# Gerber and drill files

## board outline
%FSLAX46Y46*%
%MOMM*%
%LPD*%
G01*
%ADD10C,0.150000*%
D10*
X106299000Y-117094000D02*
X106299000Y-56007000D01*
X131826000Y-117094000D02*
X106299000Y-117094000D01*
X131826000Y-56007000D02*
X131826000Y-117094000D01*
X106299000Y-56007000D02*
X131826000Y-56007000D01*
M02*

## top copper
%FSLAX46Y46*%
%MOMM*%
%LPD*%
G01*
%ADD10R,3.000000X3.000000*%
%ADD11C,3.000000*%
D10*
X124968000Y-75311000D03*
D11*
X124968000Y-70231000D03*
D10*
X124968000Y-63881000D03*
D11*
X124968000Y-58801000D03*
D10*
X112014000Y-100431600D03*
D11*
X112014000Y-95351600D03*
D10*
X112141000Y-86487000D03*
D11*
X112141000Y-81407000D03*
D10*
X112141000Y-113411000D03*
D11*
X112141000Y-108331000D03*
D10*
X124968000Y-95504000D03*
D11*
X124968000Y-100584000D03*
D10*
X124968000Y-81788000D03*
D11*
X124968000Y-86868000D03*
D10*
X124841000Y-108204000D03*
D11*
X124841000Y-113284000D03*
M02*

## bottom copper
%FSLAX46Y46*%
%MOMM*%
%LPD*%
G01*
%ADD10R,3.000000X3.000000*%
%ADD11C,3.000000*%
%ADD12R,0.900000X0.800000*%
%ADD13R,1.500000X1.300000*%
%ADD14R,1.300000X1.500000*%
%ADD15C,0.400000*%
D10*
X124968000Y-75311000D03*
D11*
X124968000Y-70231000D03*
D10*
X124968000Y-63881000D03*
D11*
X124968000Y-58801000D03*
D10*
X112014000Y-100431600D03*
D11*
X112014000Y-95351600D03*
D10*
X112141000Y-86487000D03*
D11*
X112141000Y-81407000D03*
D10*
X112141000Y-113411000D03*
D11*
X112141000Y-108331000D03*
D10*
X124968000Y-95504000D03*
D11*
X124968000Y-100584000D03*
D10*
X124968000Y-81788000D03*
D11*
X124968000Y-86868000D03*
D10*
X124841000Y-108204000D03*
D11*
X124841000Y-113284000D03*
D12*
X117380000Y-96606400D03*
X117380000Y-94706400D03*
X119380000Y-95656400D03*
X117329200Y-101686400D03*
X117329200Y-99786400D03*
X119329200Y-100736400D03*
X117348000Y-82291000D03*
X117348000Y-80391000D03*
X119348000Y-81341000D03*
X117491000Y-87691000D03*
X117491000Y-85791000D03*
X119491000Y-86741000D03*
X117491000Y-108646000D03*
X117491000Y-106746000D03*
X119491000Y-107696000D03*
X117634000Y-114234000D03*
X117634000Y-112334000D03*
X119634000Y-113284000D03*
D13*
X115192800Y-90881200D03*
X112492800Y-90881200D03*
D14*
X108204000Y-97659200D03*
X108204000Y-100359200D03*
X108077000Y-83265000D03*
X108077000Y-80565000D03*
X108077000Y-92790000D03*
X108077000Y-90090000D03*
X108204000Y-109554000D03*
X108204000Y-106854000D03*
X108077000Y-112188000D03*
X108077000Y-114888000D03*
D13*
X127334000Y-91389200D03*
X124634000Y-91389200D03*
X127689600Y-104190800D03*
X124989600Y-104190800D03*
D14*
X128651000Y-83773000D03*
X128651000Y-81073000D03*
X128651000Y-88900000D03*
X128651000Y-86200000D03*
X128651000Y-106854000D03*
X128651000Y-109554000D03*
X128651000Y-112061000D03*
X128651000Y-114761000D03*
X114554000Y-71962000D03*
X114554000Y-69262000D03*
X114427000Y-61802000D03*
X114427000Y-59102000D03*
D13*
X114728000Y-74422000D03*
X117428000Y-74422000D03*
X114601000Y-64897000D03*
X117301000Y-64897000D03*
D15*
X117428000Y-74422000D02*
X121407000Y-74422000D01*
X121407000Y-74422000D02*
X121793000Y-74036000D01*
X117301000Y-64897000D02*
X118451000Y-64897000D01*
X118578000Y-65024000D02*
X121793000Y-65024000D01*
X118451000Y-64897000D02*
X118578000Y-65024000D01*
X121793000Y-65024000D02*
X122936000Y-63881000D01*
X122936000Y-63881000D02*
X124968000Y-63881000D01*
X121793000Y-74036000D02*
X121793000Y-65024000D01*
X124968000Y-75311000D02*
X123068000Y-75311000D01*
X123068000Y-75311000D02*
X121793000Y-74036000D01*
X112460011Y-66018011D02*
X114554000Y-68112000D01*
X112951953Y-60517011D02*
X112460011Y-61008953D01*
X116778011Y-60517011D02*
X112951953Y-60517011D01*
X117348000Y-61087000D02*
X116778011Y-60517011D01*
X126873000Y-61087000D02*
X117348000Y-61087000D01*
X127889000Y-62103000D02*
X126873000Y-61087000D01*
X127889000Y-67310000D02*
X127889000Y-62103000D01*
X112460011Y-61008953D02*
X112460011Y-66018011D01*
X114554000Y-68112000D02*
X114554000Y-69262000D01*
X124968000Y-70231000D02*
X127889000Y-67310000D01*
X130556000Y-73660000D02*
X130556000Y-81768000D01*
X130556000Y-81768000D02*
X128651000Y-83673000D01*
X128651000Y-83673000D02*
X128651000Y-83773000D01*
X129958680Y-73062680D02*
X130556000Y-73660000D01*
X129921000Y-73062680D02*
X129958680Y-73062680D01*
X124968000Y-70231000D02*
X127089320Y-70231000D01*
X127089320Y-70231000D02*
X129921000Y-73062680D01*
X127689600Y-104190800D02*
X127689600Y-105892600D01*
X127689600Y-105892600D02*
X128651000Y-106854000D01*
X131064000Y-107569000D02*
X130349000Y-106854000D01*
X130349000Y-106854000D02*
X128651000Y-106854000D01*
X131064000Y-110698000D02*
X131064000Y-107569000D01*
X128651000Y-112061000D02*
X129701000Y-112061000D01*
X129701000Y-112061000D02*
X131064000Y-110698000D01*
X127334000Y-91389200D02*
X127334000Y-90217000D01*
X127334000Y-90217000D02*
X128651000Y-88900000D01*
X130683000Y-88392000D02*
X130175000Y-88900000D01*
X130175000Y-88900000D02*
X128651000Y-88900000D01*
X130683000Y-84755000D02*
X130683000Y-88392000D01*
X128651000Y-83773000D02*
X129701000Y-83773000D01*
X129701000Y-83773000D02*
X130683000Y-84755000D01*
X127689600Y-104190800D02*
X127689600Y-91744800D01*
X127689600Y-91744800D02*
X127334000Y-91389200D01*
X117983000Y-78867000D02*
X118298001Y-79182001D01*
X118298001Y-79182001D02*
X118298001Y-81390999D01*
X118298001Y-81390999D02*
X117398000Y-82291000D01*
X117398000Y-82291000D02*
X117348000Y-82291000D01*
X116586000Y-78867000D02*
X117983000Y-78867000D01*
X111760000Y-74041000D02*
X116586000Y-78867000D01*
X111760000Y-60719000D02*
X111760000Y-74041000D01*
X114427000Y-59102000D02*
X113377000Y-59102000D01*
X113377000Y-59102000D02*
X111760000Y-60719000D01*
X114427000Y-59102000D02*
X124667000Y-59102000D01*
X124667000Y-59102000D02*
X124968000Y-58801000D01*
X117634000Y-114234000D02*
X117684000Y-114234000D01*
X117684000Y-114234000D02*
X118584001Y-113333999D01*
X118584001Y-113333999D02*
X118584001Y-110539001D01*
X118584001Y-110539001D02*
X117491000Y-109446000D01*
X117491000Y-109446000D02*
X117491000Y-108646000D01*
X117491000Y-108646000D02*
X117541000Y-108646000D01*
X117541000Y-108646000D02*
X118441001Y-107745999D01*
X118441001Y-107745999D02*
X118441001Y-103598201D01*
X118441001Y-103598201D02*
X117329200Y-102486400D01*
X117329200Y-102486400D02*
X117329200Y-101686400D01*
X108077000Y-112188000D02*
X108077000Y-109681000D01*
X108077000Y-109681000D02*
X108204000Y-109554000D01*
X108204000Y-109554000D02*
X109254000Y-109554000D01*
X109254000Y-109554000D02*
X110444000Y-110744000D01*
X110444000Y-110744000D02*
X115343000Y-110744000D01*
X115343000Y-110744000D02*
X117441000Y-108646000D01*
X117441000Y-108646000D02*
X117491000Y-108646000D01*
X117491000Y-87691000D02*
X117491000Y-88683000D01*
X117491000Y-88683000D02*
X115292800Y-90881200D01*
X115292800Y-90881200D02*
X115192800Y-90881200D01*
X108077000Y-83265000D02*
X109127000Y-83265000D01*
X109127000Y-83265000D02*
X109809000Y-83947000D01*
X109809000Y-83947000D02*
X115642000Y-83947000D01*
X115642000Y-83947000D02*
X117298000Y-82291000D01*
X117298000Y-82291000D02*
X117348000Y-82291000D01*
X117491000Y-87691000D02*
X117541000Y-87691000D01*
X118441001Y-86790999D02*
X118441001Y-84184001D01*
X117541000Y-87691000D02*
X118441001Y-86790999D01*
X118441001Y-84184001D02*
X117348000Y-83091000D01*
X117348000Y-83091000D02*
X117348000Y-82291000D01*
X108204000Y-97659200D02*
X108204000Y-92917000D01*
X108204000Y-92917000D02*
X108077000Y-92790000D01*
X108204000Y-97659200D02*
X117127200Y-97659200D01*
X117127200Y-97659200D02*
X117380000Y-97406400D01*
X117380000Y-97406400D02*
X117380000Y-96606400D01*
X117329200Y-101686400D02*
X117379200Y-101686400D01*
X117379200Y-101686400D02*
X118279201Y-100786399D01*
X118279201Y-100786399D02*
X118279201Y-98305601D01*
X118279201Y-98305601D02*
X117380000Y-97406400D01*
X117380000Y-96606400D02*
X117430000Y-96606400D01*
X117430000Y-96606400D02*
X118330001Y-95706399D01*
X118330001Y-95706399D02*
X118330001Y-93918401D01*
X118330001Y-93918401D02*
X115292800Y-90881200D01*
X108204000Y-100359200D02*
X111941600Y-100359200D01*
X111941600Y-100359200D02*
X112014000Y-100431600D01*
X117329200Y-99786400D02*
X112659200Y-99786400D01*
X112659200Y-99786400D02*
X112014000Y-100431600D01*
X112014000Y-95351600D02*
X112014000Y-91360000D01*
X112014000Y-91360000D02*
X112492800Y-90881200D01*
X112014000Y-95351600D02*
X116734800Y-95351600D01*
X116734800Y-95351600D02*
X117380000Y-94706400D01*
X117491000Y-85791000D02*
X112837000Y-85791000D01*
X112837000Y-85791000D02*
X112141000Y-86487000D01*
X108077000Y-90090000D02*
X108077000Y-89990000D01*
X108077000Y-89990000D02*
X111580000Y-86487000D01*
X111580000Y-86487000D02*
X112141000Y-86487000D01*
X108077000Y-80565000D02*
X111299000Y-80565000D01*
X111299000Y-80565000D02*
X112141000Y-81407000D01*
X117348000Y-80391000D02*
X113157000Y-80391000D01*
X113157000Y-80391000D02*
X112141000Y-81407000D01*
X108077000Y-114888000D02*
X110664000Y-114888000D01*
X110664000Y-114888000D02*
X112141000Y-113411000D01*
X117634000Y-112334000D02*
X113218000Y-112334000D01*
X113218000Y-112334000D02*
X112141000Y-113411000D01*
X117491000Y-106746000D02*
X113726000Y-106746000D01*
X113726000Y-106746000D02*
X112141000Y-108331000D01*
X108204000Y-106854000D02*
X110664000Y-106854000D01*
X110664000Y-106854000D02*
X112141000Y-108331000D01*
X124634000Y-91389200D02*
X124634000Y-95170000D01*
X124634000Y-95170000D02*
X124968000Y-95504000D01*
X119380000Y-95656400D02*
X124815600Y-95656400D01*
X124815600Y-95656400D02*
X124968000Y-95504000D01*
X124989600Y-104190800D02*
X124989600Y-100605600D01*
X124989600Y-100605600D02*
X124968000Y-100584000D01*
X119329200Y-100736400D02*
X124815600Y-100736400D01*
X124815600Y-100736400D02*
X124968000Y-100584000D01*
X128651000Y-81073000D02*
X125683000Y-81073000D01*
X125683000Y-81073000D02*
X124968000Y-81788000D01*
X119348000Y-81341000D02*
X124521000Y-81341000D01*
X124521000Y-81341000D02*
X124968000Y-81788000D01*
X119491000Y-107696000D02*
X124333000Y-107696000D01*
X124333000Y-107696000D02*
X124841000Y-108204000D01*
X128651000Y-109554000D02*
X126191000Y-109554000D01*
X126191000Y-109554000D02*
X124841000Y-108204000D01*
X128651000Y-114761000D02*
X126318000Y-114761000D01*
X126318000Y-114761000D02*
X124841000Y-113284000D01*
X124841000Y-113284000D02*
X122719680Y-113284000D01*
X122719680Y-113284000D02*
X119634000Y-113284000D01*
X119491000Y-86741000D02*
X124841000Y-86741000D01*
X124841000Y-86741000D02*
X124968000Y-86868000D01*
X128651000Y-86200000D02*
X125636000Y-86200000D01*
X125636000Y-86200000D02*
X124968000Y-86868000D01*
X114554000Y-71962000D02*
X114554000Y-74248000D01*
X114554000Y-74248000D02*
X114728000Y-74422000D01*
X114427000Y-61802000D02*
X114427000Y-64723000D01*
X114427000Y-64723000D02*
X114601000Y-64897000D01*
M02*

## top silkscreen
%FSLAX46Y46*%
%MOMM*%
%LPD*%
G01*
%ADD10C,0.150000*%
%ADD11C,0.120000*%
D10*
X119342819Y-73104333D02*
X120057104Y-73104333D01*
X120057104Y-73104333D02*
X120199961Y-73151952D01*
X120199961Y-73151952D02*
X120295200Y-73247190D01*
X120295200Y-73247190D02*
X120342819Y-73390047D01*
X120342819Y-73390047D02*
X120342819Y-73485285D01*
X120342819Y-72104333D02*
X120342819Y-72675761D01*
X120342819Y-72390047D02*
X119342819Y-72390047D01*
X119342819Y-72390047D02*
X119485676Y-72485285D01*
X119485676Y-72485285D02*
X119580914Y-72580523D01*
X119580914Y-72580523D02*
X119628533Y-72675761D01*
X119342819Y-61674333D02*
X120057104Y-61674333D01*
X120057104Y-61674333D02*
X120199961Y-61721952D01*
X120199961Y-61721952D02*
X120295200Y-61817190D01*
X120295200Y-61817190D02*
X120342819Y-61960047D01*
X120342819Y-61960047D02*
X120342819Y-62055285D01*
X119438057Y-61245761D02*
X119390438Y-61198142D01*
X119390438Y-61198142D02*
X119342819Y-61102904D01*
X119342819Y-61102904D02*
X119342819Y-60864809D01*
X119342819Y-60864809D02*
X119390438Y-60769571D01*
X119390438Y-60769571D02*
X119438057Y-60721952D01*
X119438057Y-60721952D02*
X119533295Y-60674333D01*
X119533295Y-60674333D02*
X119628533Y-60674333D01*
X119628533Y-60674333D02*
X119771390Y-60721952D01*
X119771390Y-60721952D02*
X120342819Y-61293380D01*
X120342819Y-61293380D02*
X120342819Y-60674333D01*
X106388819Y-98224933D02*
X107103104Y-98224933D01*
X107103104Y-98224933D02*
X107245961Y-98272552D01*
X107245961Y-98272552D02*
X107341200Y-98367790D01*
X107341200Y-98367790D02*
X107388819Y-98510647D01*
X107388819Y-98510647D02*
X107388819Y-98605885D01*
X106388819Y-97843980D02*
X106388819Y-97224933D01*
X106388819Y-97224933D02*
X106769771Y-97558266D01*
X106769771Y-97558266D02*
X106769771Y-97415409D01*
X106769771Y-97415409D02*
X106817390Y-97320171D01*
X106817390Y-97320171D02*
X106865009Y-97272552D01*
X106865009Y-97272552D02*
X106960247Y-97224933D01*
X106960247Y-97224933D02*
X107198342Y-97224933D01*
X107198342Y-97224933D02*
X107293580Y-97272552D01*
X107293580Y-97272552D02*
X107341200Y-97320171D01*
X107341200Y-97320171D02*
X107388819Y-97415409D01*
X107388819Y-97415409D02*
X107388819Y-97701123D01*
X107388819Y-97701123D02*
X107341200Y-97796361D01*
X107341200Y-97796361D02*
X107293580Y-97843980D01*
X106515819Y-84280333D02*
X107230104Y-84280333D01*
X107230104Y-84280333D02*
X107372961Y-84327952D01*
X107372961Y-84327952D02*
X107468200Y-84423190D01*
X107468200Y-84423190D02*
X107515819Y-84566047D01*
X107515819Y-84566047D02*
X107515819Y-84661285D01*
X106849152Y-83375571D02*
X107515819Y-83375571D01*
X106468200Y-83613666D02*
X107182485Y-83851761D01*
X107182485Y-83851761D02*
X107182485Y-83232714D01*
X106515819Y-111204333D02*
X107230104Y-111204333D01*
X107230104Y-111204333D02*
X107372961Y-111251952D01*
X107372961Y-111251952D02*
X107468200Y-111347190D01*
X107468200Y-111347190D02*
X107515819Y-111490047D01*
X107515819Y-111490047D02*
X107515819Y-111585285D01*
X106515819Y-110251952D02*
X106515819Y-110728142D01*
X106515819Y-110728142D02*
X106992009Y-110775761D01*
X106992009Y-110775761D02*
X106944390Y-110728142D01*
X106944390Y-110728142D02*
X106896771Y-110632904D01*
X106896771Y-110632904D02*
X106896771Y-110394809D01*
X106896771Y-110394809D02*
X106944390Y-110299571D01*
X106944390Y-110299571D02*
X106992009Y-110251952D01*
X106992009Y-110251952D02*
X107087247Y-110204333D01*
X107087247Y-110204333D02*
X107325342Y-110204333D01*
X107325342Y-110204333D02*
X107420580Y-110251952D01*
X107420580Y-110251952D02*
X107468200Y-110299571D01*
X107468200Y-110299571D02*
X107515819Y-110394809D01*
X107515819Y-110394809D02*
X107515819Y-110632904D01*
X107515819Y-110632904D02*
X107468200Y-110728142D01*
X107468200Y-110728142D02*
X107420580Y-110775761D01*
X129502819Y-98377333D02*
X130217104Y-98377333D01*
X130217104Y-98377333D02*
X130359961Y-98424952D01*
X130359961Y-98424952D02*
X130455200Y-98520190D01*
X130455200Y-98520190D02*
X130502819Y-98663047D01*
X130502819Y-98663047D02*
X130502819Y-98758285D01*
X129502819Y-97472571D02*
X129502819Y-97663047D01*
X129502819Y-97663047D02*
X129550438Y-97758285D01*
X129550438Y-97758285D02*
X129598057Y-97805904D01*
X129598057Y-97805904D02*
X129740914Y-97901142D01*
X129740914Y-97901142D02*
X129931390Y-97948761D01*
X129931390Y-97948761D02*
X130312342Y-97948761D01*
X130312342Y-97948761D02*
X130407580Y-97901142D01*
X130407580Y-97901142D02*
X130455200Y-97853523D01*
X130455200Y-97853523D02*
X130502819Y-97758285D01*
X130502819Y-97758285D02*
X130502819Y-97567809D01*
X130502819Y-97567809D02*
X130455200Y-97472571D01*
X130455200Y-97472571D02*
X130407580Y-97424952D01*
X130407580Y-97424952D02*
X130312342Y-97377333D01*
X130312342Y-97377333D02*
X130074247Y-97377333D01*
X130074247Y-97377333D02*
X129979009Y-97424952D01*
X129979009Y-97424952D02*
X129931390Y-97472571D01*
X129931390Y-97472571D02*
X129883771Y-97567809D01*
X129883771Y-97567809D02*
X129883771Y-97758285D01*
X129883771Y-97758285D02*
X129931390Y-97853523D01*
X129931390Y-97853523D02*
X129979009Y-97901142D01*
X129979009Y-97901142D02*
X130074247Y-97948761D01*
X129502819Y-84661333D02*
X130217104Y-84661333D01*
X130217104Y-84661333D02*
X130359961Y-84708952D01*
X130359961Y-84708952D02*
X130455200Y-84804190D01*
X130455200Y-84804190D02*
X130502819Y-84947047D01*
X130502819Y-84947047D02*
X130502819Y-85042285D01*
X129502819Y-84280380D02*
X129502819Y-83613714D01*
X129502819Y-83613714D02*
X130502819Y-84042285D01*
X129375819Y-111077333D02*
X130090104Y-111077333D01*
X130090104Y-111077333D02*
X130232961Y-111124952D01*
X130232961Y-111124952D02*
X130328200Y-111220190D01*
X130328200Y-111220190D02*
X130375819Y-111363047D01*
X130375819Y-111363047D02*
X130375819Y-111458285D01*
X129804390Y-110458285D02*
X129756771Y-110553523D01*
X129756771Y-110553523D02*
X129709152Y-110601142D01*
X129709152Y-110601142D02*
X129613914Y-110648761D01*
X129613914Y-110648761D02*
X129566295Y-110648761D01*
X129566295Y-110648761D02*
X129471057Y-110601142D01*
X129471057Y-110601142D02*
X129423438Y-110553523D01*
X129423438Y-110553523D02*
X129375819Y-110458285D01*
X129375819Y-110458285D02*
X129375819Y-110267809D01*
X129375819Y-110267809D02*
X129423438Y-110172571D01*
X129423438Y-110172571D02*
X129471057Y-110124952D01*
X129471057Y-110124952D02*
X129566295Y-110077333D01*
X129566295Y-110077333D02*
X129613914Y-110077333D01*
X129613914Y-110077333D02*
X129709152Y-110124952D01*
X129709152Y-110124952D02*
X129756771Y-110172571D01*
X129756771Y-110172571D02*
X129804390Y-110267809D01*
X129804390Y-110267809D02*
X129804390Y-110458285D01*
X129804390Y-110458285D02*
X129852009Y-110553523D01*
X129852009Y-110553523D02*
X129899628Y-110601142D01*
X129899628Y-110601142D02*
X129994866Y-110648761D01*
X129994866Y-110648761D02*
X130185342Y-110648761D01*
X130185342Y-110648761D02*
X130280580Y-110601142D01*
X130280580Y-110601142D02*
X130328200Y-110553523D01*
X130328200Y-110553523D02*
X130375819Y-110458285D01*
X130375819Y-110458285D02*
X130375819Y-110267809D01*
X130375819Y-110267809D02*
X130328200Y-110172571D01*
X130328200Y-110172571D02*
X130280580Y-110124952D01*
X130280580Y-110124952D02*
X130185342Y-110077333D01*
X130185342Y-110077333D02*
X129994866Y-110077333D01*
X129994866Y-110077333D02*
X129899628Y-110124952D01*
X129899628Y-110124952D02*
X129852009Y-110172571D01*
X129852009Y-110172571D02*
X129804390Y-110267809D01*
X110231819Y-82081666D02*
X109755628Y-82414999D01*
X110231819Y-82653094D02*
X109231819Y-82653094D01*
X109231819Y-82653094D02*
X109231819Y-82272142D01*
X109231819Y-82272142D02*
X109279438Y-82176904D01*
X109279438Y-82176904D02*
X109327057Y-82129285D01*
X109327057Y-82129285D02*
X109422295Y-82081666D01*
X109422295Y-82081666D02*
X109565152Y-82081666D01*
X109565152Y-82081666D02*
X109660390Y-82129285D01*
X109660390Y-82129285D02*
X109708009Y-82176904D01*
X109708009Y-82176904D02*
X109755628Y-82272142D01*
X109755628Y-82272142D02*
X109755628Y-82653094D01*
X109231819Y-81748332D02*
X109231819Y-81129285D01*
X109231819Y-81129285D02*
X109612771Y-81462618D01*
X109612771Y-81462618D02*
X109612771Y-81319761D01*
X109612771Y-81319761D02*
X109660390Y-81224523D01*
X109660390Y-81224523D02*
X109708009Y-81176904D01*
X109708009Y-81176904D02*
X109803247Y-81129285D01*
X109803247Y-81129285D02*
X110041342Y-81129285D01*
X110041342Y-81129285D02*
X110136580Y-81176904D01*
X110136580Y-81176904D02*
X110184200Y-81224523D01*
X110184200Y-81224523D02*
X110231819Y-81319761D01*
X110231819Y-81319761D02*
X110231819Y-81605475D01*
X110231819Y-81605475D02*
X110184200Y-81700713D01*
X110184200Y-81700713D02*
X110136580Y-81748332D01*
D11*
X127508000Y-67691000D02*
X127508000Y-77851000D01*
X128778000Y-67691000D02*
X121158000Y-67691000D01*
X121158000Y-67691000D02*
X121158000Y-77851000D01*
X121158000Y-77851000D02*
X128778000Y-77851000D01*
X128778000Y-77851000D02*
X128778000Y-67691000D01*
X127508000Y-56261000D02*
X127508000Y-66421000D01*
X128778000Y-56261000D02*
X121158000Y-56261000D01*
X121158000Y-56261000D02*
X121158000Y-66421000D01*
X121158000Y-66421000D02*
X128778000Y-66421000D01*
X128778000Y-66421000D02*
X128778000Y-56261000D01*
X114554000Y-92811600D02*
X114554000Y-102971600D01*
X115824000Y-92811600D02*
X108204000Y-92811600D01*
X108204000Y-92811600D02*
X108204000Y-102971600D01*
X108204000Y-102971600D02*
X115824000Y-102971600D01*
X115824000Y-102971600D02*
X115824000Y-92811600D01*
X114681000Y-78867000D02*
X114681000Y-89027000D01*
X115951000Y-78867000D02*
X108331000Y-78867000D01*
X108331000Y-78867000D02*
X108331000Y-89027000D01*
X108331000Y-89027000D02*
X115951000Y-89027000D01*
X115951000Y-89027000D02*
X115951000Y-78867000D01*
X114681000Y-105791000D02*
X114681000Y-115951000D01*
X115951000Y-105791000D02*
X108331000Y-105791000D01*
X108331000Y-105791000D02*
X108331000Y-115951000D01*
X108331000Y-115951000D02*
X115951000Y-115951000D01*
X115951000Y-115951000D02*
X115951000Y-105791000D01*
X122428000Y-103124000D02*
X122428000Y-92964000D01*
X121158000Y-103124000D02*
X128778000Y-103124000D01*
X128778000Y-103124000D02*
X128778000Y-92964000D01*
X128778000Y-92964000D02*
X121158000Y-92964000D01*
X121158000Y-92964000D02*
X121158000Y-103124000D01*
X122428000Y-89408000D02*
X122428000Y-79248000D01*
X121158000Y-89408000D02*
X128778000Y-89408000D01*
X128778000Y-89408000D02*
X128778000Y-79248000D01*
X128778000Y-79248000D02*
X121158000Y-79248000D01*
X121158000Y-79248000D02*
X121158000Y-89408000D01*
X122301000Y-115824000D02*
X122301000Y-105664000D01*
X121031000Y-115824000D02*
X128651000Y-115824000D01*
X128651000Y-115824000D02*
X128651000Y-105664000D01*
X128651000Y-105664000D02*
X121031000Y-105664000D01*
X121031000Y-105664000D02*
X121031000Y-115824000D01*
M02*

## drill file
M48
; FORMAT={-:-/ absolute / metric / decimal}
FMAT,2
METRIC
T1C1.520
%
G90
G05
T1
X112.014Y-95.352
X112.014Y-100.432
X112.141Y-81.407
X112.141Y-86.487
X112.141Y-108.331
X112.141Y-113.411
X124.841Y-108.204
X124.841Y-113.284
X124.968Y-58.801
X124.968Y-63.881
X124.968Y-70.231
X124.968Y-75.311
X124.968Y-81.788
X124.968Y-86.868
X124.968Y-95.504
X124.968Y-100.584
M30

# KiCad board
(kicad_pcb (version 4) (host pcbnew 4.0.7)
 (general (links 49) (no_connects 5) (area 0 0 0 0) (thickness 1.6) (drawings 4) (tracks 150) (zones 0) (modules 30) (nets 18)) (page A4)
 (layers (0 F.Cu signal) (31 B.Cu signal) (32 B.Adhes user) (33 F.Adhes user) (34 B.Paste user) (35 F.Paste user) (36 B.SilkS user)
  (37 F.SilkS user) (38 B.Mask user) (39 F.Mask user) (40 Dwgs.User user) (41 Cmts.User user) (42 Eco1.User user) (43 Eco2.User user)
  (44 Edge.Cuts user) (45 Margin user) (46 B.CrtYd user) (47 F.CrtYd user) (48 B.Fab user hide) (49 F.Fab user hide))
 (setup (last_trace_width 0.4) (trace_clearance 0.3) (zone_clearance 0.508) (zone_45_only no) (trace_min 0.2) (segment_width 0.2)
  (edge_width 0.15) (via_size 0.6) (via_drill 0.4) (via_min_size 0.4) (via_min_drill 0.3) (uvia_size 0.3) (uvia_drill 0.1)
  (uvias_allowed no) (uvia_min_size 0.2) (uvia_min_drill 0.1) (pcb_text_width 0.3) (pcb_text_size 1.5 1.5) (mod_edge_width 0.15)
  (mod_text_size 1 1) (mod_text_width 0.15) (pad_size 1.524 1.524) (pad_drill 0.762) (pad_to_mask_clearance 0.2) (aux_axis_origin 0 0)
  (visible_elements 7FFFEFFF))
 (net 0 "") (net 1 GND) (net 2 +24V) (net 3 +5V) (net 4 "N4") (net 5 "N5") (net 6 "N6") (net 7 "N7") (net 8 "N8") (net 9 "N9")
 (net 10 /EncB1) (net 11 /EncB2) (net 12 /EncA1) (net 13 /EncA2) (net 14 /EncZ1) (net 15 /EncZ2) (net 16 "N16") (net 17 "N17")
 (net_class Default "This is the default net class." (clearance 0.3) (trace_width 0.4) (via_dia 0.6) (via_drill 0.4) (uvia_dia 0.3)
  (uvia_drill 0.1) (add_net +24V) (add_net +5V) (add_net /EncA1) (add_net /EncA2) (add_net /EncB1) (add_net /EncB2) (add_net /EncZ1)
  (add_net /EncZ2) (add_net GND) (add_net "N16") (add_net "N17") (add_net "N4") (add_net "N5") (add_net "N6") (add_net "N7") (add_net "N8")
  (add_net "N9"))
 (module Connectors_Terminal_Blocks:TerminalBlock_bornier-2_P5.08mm (layer F.Cu) (at 124.968 75.311 90)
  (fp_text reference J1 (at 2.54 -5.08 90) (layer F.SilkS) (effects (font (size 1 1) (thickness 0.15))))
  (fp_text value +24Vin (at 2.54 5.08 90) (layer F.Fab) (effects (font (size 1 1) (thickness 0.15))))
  (fp_line (start 7.62 2.54) (end -2.54 2.54) (layer F.SilkS) (width 0.12))
  (fp_line (start 7.62 3.81) (end 7.62 -3.81) (layer F.SilkS) (width 0.12))
  (fp_line (start 7.62 -3.81) (end -2.54 -3.81) (layer F.SilkS) (width 0.12))
  (fp_line (start -2.54 -3.81) (end -2.54 3.81) (layer F.SilkS) (width 0.12))
  (fp_line (start -2.54 3.81) (end 7.62 3.81) (layer F.SilkS) (width 0.12))
  (pad 1 thru_hole rect (at 0 0 90) (size 3 3) (drill 1.52) (layers *.Cu *.Mask) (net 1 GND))
  (pad 2 thru_hole circle (at 5.08 0 90) (size 3 3) (drill 1.52) (layers *.Cu *.Mask) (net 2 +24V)))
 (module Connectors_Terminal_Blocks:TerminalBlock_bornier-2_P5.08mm (layer F.Cu) (at 124.968 63.881 90)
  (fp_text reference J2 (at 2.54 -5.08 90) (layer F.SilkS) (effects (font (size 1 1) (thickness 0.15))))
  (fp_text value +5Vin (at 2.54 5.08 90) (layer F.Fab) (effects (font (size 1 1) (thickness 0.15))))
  (fp_line (start 7.62 2.54) (end -2.54 2.54) (layer F.SilkS) (width 0.12))
  (fp_line (start 7.62 3.81) (end 7.62 -3.81) (layer F.SilkS) (width 0.12))
  (fp_line (start 7.62 -3.81) (end -2.54 -3.81) (layer F.SilkS) (width 0.12))
  (fp_line (start -2.54 -3.81) (end -2.54 3.81) (layer F.SilkS) (width 0.12))
  (fp_line (start -2.54 3.81) (end 7.62 3.81) (layer F.SilkS) (width 0.12))
  (pad 1 thru_hole rect (at 0 0 90) (size 3 3) (drill 1.52) (layers *.Cu *.Mask) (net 1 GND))
  (pad 2 thru_hole circle (at 5.08 0 90) (size 3 3) (drill 1.52) (layers *.Cu *.Mask) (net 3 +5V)))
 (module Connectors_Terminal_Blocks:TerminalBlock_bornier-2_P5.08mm (layer F.Cu) (at 112.014 100.4316 90)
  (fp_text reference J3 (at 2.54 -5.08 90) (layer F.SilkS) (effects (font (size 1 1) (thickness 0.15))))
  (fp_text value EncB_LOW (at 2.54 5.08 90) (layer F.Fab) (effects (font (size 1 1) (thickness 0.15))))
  (fp_line (start 7.62 2.54) (end -2.54 2.54) (layer F.SilkS) (width 0.12))
  (fp_line (start 7.62 3.81) (end 7.62 -3.81) (layer F.SilkS) (width 0.12))
  (fp_line (start 7.62 -3.81) (end -2.54 -3.81) (layer F.SilkS) (width 0.12))
  (fp_line (start -2.54 -3.81) (end -2.54 3.81) (layer F.SilkS) (width 0.12))
  (fp_line (start -2.54 3.81) (end 7.62 3.81) (layer F.SilkS) (width 0.12))
  (pad 1 thru_hole rect (at 0 0 90) (size 3 3) (drill 1.52) (layers *.Cu *.Mask) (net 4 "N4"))
  (pad 2 thru_hole circle (at 5.08 0 90) (size 3 3) (drill 1.52) (layers *.Cu *.Mask) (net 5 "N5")))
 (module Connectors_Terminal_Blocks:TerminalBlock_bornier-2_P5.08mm (layer F.Cu) (at 112.141 86.487 90)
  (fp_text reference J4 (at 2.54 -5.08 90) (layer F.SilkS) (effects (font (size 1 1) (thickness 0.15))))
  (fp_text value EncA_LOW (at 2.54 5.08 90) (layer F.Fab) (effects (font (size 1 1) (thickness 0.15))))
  (fp_line (start 7.62 2.54) (end -2.54 2.54) (layer F.SilkS) (width 0.12))
  (fp_line (start 7.62 3.81) (end 7.62 -3.81) (layer F.SilkS) (width 0.12))
  (fp_line (start 7.62 -3.81) (end -2.54 -3.81) (layer F.SilkS) (width 0.12))
  (fp_line (start -2.54 -3.81) (end -2.54 3.81) (layer F.SilkS) (width 0.12))
  (fp_line (start -2.54 3.81) (end 7.62 3.81) (layer F.SilkS) (width 0.12))
  (pad 1 thru_hole rect (at 0 0 90) (size 3 3) (drill 1.52) (layers *.Cu *.Mask) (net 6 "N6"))
  (pad 2 thru_hole circle (at 5.08 0 90) (size 3 3) (drill 1.52) (layers *.Cu *.Mask) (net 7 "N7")))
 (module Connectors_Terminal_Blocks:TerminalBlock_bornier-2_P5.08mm (layer F.Cu) (at 112.141 113.411 90)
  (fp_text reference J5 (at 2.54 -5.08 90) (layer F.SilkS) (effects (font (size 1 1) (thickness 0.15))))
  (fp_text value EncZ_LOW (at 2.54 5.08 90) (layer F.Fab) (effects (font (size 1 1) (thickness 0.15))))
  (fp_line (start 7.62 2.54) (end -2.54 2.54) (layer F.SilkS) (width 0.12))
  (fp_line (start 7.62 3.81) (end 7.62 -3.81) (layer F.SilkS) (width 0.12))
  (fp_line (start 7.62 -3.81) (end -2.54 -3.81) (layer F.SilkS) (width 0.12))
  (fp_line (start -2.54 -3.81) (end -2.54 3.81) (layer F.SilkS) (width 0.12))
  (fp_line (start -2.54 3.81) (end 7.62 3.81) (layer F.SilkS) (width 0.12))
  (pad 1 thru_hole rect (at 0 0 90) (size 3 3) (drill 1.52) (layers *.Cu *.Mask) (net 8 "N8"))
  (pad 2 thru_hole circle (at 5.08 0 90) (size 3 3) (drill 1.52) (layers *.Cu *.Mask) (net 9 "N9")))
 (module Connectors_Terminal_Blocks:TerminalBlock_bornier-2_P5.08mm (layer F.Cu) (at 124.968 95.504 270)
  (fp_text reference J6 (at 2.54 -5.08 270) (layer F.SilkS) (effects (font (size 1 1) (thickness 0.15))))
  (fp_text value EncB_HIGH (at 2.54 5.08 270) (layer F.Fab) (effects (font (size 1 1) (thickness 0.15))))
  (fp_line (start 7.62 2.54) (end -2.54 2.54) (layer F.SilkS) (width 0.12))
  (fp_line (start 7.62 3.81) (end 7.62 -3.81) (layer F.SilkS) (width 0.12))
  (fp_line (start 7.62 -3.81) (end -2.54 -3.81) (layer F.SilkS) (width 0.12))
  (fp_line (start -2.54 -3.81) (end -2.54 3.81) (layer F.SilkS) (width 0.12))
  (fp_line (start -2.54 3.81) (end 7.62 3.81) (layer F.SilkS) (width 0.12))
  (pad 1 thru_hole rect (at 0 0 270) (size 3 3) (drill 1.52) (layers *.Cu *.Mask) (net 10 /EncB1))
  (pad 2 thru_hole circle (at 5.08 0 270) (size 3 3) (drill 1.52) (layers *.Cu *.Mask) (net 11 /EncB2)))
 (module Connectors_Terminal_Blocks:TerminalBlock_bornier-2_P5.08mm (layer F.Cu) (at 124.968 81.788 270)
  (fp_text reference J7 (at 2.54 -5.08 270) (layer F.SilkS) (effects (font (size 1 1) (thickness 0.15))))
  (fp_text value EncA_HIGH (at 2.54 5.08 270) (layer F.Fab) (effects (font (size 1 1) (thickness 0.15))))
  (fp_line (start 7.62 2.54) (end -2.54 2.54) (layer F.SilkS) (width 0.12))
  (fp_line (start 7.62 3.81) (end 7.62 -3.81) (layer F.SilkS) (width 0.12))
  (fp_line (start 7.62 -3.81) (end -2.54 -3.81) (layer F.SilkS) (width 0.12))
  (fp_line (start -2.54 -3.81) (end -2.54 3.81) (layer F.SilkS) (width 0.12))
  (fp_line (start -2.54 3.81) (end 7.62 3.81) (layer F.SilkS) (width 0.12))
  (pad 1 thru_hole rect (at 0 0 270) (size 3 3) (drill 1.52) (layers *.Cu *.Mask) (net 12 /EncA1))
  (pad 2 thru_hole circle (at 5.08 0 270) (size 3 3) (drill 1.52) (layers *.Cu *.Mask) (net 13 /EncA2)))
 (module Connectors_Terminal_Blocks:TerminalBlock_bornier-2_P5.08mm (layer F.Cu) (at 124.841 108.204 270)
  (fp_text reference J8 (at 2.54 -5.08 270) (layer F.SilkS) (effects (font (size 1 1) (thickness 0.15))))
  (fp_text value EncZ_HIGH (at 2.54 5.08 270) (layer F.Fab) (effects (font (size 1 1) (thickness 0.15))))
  (fp_line (start 7.62 2.54) (end -2.54 2.54) (layer F.SilkS) (width 0.12))
  (fp_line (start 7.62 3.81) (end 7.62 -3.81) (layer F.SilkS) (width 0.12))
  (fp_line (start 7.62 -3.81) (end -2.54 -3.81) (layer F.SilkS) (width 0.12))
  (fp_line (start -2.54 -3.81) (end -2.54 3.81) (layer F.SilkS) (width 0.12))
  (fp_line (start -2.54 3.81) (end 7.62 3.81) (layer F.SilkS) (width 0.12))
  (pad 1 thru_hole rect (at 0 0 270) (size 3 3) (drill 1.52) (layers *.Cu *.Mask) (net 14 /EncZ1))
  (pad 2 thru_hole circle (at 5.08 0 270) (size 3 3) (drill 1.52) (layers *.Cu *.Mask) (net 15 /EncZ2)))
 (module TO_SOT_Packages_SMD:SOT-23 (layer B.Cu) (at 118.38 95.6564)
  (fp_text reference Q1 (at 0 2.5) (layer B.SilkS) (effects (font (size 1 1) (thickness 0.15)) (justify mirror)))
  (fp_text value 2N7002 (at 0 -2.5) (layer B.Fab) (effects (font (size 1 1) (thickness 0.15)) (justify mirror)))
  (pad 1 smd rect (at -1 0.95) (size 0.9 0.8) (layers B.Cu B.Paste B.Mask) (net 3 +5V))
  (pad 2 smd rect (at -1 -0.95) (size 0.9 0.8) (layers B.Cu B.Paste B.Mask) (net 5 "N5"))
  (pad 3 smd rect (at 1 0) (size 0.9 0.8) (layers B.Cu B.Paste B.Mask) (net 10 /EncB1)))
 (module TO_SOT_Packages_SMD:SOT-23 (layer B.Cu) (at 118.3292 100.7364)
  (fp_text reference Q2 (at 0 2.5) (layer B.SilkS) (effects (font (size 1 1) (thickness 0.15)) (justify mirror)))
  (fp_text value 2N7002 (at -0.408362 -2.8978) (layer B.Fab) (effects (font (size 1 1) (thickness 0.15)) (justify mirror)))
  (pad 1 smd rect (at -1 0.95) (size 0.9 0.8) (layers B.Cu B.Paste B.Mask) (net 3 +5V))
  (pad 2 smd rect (at -1 -0.95) (size 0.9 0.8) (layers B.Cu B.Paste B.Mask) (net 4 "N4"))
  (pad 3 smd rect (at 1 0) (size 0.9 0.8) (layers B.Cu B.Paste B.Mask) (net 11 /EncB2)))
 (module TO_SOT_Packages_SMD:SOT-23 (layer B.Cu) (at 118.348 81.341)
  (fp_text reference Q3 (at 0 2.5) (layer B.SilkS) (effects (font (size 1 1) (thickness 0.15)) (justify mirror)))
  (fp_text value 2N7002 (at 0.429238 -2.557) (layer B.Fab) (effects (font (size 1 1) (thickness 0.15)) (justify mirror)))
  (pad 1 smd rect (at -1 0.95) (size 0.9 0.8) (layers B.Cu B.Paste B.Mask) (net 3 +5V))
  (pad 2 smd rect (at -1 -0.95) (size 0.9 0.8) (layers B.Cu B.Paste B.Mask) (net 7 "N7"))
  (pad 3 smd rect (at 1 0) (size 0.9 0.8) (layers B.Cu B.Paste B.Mask) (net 12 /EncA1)))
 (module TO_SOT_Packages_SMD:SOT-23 (layer B.Cu) (at 118.491 86.741)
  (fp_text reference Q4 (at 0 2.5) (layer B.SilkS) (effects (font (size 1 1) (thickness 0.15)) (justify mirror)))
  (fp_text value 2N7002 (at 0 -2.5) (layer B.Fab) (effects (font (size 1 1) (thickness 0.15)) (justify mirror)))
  (pad 1 smd rect (at -1 0.95) (size 0.9 0.8) (layers B.Cu B.Paste B.Mask) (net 3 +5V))
  (pad 2 smd rect (at -1 -0.95) (size 0.9 0.8) (layers B.Cu B.Paste B.Mask) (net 6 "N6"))
  (pad 3 smd rect (at 1 0) (size 0.9 0.8) (layers B.Cu B.Paste B.Mask) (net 13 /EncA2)))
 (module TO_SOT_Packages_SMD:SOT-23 (layer B.Cu) (at 118.491 107.696)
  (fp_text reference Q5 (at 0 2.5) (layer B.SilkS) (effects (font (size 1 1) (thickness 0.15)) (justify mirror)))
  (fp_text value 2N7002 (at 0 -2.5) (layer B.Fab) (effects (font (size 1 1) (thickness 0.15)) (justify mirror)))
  (pad 1 smd rect (at -1 0.95) (size 0.9 0.8) (layers B.Cu B.Paste B.Mask) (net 3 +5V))
  (pad 2 smd rect (at -1 -0.95) (size 0.9 0.8) (layers B.Cu B.Paste B.Mask) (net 9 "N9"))
  (pad 3 smd rect (at 1 0) (size 0.9 0.8) (layers B.Cu B.Paste B.Mask) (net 14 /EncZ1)))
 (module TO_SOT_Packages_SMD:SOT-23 (layer B.Cu) (at 118.634 113.284)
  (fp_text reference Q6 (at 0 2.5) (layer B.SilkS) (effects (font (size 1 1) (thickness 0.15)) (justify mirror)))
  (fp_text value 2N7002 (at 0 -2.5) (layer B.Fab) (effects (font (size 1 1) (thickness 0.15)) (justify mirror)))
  (pad 1 smd rect (at -1 0.95) (size 0.9 0.8) (layers B.Cu B.Paste B.Mask) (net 3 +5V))
  (pad 2 smd rect (at -1 -0.95) (size 0.9 0.8) (layers B.Cu B.Paste B.Mask) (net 8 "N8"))
  (pad 3 smd rect (at 1 0) (size 0.9 0.8) (layers B.Cu B.Paste B.Mask) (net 15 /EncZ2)))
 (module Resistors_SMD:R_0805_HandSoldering (layer B.Cu) (at 113.8428 90.8812 180)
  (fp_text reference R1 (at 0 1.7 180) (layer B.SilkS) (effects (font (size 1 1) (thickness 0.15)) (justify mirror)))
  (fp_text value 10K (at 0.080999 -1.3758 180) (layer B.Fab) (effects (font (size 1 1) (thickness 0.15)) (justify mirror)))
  (pad 1 smd rect (at -1.35 0 180) (size 1.5 1.3) (layers B.Cu B.Paste B.Mask) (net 3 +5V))
  (pad 2 smd rect (at 1.35 0 180) (size 1.5 1.3) (layers B.Cu B.Paste B.Mask) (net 5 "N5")))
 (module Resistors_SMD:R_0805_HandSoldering (layer B.Cu) (at 108.204 99.0092 270)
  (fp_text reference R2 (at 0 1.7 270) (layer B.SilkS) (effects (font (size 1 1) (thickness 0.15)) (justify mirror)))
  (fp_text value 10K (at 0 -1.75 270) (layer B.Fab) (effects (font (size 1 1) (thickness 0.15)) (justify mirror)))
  (pad 1 smd rect (at -1.35 0 270) (size 1.5 1.3) (layers B.Cu B.Paste B.Mask) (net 3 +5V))
  (pad 2 smd rect (at 1.35 0 270) (size 1.5 1.3) (layers B.Cu B.Paste B.Mask) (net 4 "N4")))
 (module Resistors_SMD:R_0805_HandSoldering (layer B.Cu) (at 108.077 81.915 90)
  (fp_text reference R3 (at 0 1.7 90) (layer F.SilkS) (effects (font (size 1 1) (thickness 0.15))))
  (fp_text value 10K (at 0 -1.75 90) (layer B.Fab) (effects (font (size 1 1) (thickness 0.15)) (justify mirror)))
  (pad 1 smd rect (at -1.35 0 90) (size 1.5 1.3) (layers B.Cu B.Paste B.Mask) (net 3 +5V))
  (pad 2 smd rect (at 1.35 0 90) (size 1.5 1.3) (layers B.Cu B.Paste B.Mask) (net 7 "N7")))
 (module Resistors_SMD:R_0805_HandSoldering (layer B.Cu) (at 108.077 91.44 90)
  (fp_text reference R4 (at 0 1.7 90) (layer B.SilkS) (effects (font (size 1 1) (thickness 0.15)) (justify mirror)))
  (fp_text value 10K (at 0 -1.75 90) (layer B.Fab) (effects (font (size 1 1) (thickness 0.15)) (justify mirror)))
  (pad 1 smd rect (at -1.35 0 90) (size 1.5 1.3) (layers B.Cu B.Paste B.Mask) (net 3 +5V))
  (pad 2 smd rect (at 1.35 0 90) (size 1.5 1.3) (layers B.Cu B.Paste B.Mask) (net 6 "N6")))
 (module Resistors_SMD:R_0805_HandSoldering (layer B.Cu) (at 108.204 108.204 90)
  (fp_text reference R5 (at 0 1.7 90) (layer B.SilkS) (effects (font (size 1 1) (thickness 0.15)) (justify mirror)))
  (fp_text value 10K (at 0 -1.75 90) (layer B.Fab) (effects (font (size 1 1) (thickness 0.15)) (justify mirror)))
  (pad 1 smd rect (at -1.35 0 90) (size 1.5 1.3) (layers B.Cu B.Paste B.Mask) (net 3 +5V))
  (pad 2 smd rect (at 1.35 0 90) (size 1.5 1.3) (layers B.Cu B.Paste B.Mask) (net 9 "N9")))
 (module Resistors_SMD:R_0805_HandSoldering (layer B.Cu) (at 108.077 113.538 270)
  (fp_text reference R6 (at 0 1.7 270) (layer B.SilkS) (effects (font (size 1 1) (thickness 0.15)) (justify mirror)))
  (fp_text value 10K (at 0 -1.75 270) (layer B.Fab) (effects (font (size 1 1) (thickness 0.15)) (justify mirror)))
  (pad 1 smd rect (at -1.35 0 270) (size 1.5 1.3) (layers B.Cu B.Paste B.Mask) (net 3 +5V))
  (pad 2 smd rect (at 1.35 0 270) (size 1.5 1.3) (layers B.Cu B.Paste B.Mask) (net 8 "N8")))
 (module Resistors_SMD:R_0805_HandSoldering (layer B.Cu) (at 125.984 91.3892 180)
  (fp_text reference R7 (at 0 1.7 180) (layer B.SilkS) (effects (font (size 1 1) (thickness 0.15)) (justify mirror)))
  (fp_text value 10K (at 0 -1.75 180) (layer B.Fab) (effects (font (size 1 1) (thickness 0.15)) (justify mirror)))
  (pad 1 smd rect (at -1.35 0 180) (size 1.5 1.3) (layers B.Cu B.Paste B.Mask) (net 2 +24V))
  (pad 2 smd rect (at 1.35 0 180) (size 1.5 1.3) (layers B.Cu B.Paste B.Mask) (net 10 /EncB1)))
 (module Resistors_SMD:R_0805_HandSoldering (layer B.Cu) (at 126.3396 104.1908 180)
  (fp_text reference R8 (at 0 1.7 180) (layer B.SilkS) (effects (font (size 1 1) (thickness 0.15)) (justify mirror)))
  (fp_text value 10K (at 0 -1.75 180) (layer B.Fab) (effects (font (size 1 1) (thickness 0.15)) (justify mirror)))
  (pad 1 smd rect (at -1.35 0 180) (size 1.5 1.3) (layers B.Cu B.Paste B.Mask) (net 2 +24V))
  (pad 2 smd rect (at 1.35 0 180) (size 1.5 1.3) (layers B.Cu B.Paste B.Mask) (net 11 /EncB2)))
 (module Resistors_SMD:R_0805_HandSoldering (layer B.Cu) (at 128.651 82.423 90)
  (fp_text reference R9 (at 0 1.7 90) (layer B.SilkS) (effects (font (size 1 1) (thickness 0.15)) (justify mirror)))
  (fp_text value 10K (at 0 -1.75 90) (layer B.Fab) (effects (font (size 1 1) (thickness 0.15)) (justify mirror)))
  (pad 1 smd rect (at -1.35 0 90) (size 1.5 1.3) (layers B.Cu B.Paste B.Mask) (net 2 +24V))
  (pad 2 smd rect (at 1.35 0 90) (size 1.5 1.3) (layers B.Cu B.Paste B.Mask) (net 12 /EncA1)))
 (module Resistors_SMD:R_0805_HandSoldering (layer B.Cu) (at 128.651 87.55 90)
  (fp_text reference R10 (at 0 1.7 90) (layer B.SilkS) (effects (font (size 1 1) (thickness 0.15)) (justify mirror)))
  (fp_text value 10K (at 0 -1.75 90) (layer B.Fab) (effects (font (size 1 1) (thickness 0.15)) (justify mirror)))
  (pad 1 smd rect (at -1.35 0 90) (size 1.5 1.3) (layers B.Cu B.Paste B.Mask) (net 2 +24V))
  (pad 2 smd rect (at 1.35 0 90) (size 1.5 1.3) (layers B.Cu B.Paste B.Mask) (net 13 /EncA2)))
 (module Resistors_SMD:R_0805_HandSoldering (layer B.Cu) (at 128.651 108.204 270)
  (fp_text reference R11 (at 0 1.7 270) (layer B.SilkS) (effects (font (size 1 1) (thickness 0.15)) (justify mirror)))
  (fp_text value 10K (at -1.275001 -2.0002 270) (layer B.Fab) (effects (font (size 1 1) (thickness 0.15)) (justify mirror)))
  (pad 1 smd rect (at -1.35 0 270) (size 1.5 1.3) (layers B.Cu B.Paste B.Mask) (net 2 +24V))
  (pad 2 smd rect (at 1.35 0 270) (size 1.5 1.3) (layers B.Cu B.Paste B.Mask) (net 14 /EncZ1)))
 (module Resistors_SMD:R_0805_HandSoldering (layer B.Cu) (at 128.651 113.411 270)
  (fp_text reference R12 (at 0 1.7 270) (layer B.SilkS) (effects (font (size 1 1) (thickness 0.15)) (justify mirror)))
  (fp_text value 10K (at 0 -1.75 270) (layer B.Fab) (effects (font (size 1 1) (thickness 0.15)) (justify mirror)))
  (pad 1 smd rect (at -1.35 0 270) (size 1.5 1.3) (layers B.Cu B.Paste B.Mask) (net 2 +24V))
  (pad 2 smd rect (at 1.35 0 270) (size 1.5 1.3) (layers B.Cu B.Paste B.Mask) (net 15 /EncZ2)))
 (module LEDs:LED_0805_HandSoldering (layer B.Cu) (at 114.554 70.612 90)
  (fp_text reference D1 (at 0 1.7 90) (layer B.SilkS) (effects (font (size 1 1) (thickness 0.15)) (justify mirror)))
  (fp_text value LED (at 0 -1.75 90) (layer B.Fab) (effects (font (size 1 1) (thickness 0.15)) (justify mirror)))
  (pad 1 smd rect (at -1.35 0 90) (size 1.5 1.3) (layers B.Cu B.Paste B.Mask) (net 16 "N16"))
  (pad 2 smd rect (at 1.35 0 90) (size 1.5 1.3) (layers B.Cu B.Paste B.Mask) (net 2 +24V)))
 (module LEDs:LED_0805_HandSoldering (layer B.Cu) (at 114.427 60.452 90)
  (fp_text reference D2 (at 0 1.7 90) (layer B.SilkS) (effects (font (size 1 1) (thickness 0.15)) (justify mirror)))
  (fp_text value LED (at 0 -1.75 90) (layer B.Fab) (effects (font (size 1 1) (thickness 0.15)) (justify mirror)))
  (pad 1 smd rect (at -1.35 0 90) (size 1.5 1.3) (layers B.Cu B.Paste B.Mask) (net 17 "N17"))
  (pad 2 smd rect (at 1.35 0 90) (size 1.5 1.3) (layers B.Cu B.Paste B.Mask) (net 3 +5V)))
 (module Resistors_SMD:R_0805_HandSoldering (layer B.Cu) (at 116.078 74.422)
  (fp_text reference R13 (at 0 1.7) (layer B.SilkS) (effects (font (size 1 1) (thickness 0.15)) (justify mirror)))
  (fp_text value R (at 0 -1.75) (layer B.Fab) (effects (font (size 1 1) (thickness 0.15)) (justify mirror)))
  (pad 1 smd rect (at -1.35 0) (size 1.5 1.3) (layers B.Cu B.Paste B.Mask) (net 16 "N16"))
  (pad 2 smd rect (at 1.35 0) (size 1.5 1.3) (layers B.Cu B.Paste B.Mask) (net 1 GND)))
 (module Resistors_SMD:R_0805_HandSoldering (layer B.Cu) (at 115.951 64.897)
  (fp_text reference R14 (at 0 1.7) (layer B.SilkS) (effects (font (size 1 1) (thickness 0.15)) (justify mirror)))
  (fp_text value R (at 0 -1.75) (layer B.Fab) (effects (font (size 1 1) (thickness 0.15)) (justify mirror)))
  (pad 1 smd rect (at -1.35 0) (size 1.5 1.3) (layers B.Cu B.Paste B.Mask) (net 17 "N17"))
  (pad 2 smd rect (at 1.35 0) (size 1.5 1.3) (layers B.Cu B.Paste B.Mask) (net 1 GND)))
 (gr_line (start 106.299 117.094) (end 106.299 56.007) (layer Edge.Cuts) (width 0.15))
 (gr_line (start 131.826 117.094) (end 106.299 117.094) (layer Edge.Cuts) (width 0.15))
 (gr_line (start 131.826 56.007) (end 131.826 117.094) (layer Edge.Cuts) (width 0.15))
 (gr_line (start 106.299 56.007) (end 131.826 56.007) (layer Edge.Cuts) (width 0.15))
 (segment (start 117.428 74.422) (end 121.407 74.422) (width 0.4) (layer B.Cu) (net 1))
 (segment (start 121.407 74.422) (end 121.793 74.036) (width 0.4) (layer B.Cu) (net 1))
 (segment (start 117.301 64.897) (end 118.451 64.897) (width 0.4) (layer B.Cu) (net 1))
 (segment (start 118.578 65.024) (end 121.793 65.024) (width 0.4) (layer B.Cu) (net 1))
 (segment (start 118.451 64.897) (end 118.578 65.024) (width 0.4) (layer B.Cu) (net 1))
 (segment (start 121.793 65.024) (end 122.936 63.881) (width 0.4) (layer B.Cu) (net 1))
 (segment (start 122.936 63.881) (end 124.968 63.881) (width 0.4) (layer B.Cu) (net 1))
 (segment (start 121.793 74.036) (end 121.793 65.024) (width 0.4) (layer B.Cu) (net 1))
 (segment (start 124.968 75.311) (end 123.068 75.311) (width 0.4) (layer B.Cu) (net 1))
 (segment (start 123.068 75.311) (end 121.793 74.036) (width 0.4) (layer B.Cu) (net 1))
 (segment (start 112.460011 66.018011) (end 114.554 68.112) (width 0.4) (layer B.Cu) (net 2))
 (segment (start 112.951953 60.517011) (end 112.460011 61.008953) (width 0.4) (layer B.Cu) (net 2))
 (segment (start 116.778011 60.517011) (end 112.951953 60.517011) (width 0.4) (layer B.Cu) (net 2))
 (segment (start 117.348 61.087) (end 116.778011 60.517011) (width 0.4) (layer B.Cu) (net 2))
 (segment (start 126.873 61.087) (end 117.348 61.087) (width 0.4) (layer B.Cu) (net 2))
 (segment (start 127.889 62.103) (end 126.873 61.087) (width 0.4) (layer B.Cu) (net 2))
 (segment (start 127.889 67.31) (end 127.889 62.103) (width 0.4) (layer B.Cu) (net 2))
 (segment (start 112.460011 61.008953) (end 112.460011 66.018011) (width 0.4) (layer B.Cu) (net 2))
 (segment (start 114.554 68.112) (end 114.554 69.262) (width 0.4) (layer B.Cu) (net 2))
 (segment (start 124.968 70.231) (end 127.889 67.31) (width 0.4) (layer B.Cu) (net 2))
 (segment (start 130.556 73.66) (end 130.556 81.768) (width 0.4) (layer B.Cu) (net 2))
 (segment (start 130.556 81.768) (end 128.651 83.673) (width 0.4) (layer B.Cu) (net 2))
 (segment (start 128.651 83.673) (end 128.651 83.773) (width 0.4) (layer B.Cu) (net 2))
 (segment (start 129.95868 73.06268) (end 130.556 73.66) (width 0.4) (layer B.Cu) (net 2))
 (segment (start 129.921 73.06268) (end 129.95868 73.06268) (width 0.4) (layer B.Cu) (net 2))
 (segment (start 124.968 70.231) (end 127.08932 70.231) (width 0.4) (layer B.Cu) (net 2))
 (segment (start 127.08932 70.231) (end 129.921 73.06268) (width 0.4) (layer B.Cu) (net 2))
 (segment (start 127.6896 104.1908) (end 127.6896 105.8926) (width 0.4) (layer B.Cu) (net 2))
 (segment (start 127.6896 105.8926) (end 128.651 106.854) (width 0.4) (layer B.Cu) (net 2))
 (segment (start 131.064 107.569) (end 130.349 106.854) (width 0.4) (layer B.Cu) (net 2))
 (segment (start 130.349 106.854) (end 128.651 106.854) (width 0.4) (layer B.Cu) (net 2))
 (segment (start 131.064 110.698) (end 131.064 107.569) (width 0.4) (layer B.Cu) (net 2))
 (segment (start 128.651 112.061) (end 129.701 112.061) (width 0.4) (layer B.Cu) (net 2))
 (segment (start 129.701 112.061) (end 131.064 110.698) (width 0.4) (layer B.Cu) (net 2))
 (segment (start 127.334 91.3892) (end 127.334 90.217) (width 0.4) (layer B.Cu) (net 2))
 (segment (start 127.334 90.217) (end 128.651 88.9) (width 0.4) (layer B.Cu) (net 2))
 (segment (start 130.683 88.392) (end 130.175 88.9) (width 0.4) (layer B.Cu) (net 2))
 (segment (start 130.175 88.9) (end 128.651 88.9) (width 0.4) (layer B.Cu) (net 2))
 (segment (start 130.683 84.755) (end 130.683 88.392) (width 0.4) (layer B.Cu) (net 2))
 (segment (start 128.651 83.773) (end 129.701 83.773) (width 0.4) (layer B.Cu) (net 2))
 (segment (start 129.701 83.773) (end 130.683 84.755) (width 0.4) (layer B.Cu) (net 2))
 (segment (start 127.6896 104.1908) (end 127.6896 91.7448) (width 0.4) (layer B.Cu) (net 2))
 (segment (start 127.6896 91.7448) (end 127.334 91.3892) (width 0.4) (layer B.Cu) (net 2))
 (segment (start 117.983 78.867) (end 118.298001 79.182001) (width 0.4) (layer B.Cu) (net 3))
 (segment (start 118.298001 79.182001) (end 118.298001 81.390999) (width 0.4) (layer B.Cu) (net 3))
 (segment (start 118.298001 81.390999) (end 117.398 82.291) (width 0.4) (layer B.Cu) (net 3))
 (segment (start 117.398 82.291) (end 117.348 82.291) (width 0.4) (layer B.Cu) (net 3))
 (segment (start 116.586 78.867) (end 117.983 78.867) (width 0.4) (layer B.Cu) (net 3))
 (segment (start 111.76 74.041) (end 116.586 78.867) (width 0.4) (layer B.Cu) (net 3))
 (segment (start 111.76 60.719) (end 111.76 74.041) (width 0.4) (layer B.Cu) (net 3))
 (segment (start 114.427 59.102) (end 113.377 59.102) (width 0.4) (layer B.Cu) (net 3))
 (segment (start 113.377 59.102) (end 111.76 60.719) (width 0.4) (layer B.Cu) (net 3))
 (segment (start 114.427 59.102) (end 124.667 59.102) (width 0.4) (layer B.Cu) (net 3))
 (segment (start 124.667 59.102) (end 124.968 58.801) (width 0.4) (layer B.Cu) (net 3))
 (segment (start 117.634 114.234) (end 117.684 114.234) (width 0.4) (layer B.Cu) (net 3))
 (segment (start 117.684 114.234) (end 118.584001 113.333999) (width 0.4) (layer B.Cu) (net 3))
 (segment (start 118.584001 113.333999) (end 118.584001 110.539001) (width 0.4) (layer B.Cu) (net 3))
 (segment (start 118.584001 110.539001) (end 117.491 109.446) (width 0.4) (layer B.Cu) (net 3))
 (segment (start 117.491 109.446) (end 117.491 108.646) (width 0.4) (layer B.Cu) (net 3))
 (segment (start 117.491 108.646) (end 117.541 108.646) (width 0.4) (layer B.Cu) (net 3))
 (segment (start 117.541 108.646) (end 118.441001 107.745999) (width 0.4) (layer B.Cu) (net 3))
 (segment (start 118.441001 107.745999) (end 118.441001 103.598201) (width 0.4) (layer B.Cu) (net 3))
 (segment (start 118.441001 103.598201) (end 117.3292 102.4864) (width 0.4) (layer B.Cu) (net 3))
 (segment (start 117.3292 102.4864) (end 117.3292 101.6864) (width 0.4) (layer B.Cu) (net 3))
 (segment (start 108.077 112.188) (end 108.077 109.681) (width 0.4) (layer B.Cu) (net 3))
 (segment (start 108.077 109.681) (end 108.204 109.554) (width 0.4) (layer B.Cu) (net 3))
 (segment (start 108.204 109.554) (end 109.254 109.554) (width 0.4) (layer B.Cu) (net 3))
 (segment (start 109.254 109.554) (end 110.444 110.744) (width 0.4) (layer B.Cu) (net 3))
 (segment (start 110.444 110.744) (end 115.343 110.744) (width 0.4) (layer B.Cu) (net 3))
 (segment (start 115.343 110.744) (end 117.441 108.646) (width 0.4) (layer B.Cu) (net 3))
 (segment (start 117.441 108.646) (end 117.491 108.646) (width 0.4) (layer B.Cu) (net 3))
 (segment (start 117.491 87.691) (end 117.491 88.683) (width 0.4) (layer B.Cu) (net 3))
 (segment (start 117.491 88.683) (end 115.2928 90.8812) (width 0.4) (layer B.Cu) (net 3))
 (segment (start 115.2928 90.8812) (end 115.1928 90.8812) (width 0.4) (layer B.Cu) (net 3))
 (segment (start 108.077 83.265) (end 109.127 83.265) (width 0.4) (layer B.Cu) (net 3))
 (segment (start 109.127 83.265) (end 109.809 83.947) (width 0.4) (layer B.Cu) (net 3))
 (segment (start 109.809 83.947) (end 115.642 83.947) (width 0.4) (layer B.Cu) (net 3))
 (segment (start 115.642 83.947) (end 117.298 82.291) (width 0.4) (layer B.Cu) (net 3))
 (segment (start 117.298 82.291) (end 117.348 82.291) (width 0.4) (layer B.Cu) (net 3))
 (segment (start 117.491 87.691) (end 117.541 87.691) (width 0.4) (layer B.Cu) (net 3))
 (segment (start 118.441001 86.790999) (end 118.441001 84.184001) (width 0.4) (layer B.Cu) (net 3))
 (segment (start 117.541 87.691) (end 118.441001 86.790999) (width 0.4) (layer B.Cu) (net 3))
 (segment (start 118.441001 84.184001) (end 117.348 83.091) (width 0.4) (layer B.Cu) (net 3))
 (segment (start 117.348 83.091) (end 117.348 82.291) (width 0.4) (layer B.Cu) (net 3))
 (segment (start 108.204 97.6592) (end 108.204 92.917) (width 0.4) (layer B.Cu) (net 3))
 (segment (start 108.204 92.917) (end 108.077 92.79) (width 0.4) (layer B.Cu) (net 3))
 (segment (start 108.204 97.6592) (end 117.1272 97.6592) (width 0.4) (layer B.Cu) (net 3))
 (segment (start 117.1272 97.6592) (end 117.38 97.4064) (width 0.4) (layer B.Cu) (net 3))
 (segment (start 117.38 97.4064) (end 117.38 96.6064) (width 0.4) (layer B.Cu) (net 3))
 (segment (start 117.3292 101.6864) (end 117.3792 101.6864) (width 0.4) (layer B.Cu) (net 3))
 (segment (start 117.3792 101.6864) (end 118.279201 100.786399) (width 0.4) (layer B.Cu) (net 3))
 (segment (start 118.279201 100.786399) (end 118.279201 98.305601) (width 0.4) (layer B.Cu) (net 3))
 (segment (start 118.279201 98.305601) (end 117.38 97.4064) (width 0.4) (layer B.Cu) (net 3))
 (segment (start 117.38 96.6064) (end 117.43 96.6064) (width 0.4) (layer B.Cu) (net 3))
 (segment (start 117.43 96.6064) (end 118.330001 95.706399) (width 0.4) (layer B.Cu) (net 3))
 (segment (start 118.330001 95.706399) (end 118.330001 93.918401) (width 0.4) (layer B.Cu) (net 3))
 (segment (start 118.330001 93.918401) (end 115.2928 90.8812) (width 0.4) (layer B.Cu) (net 3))
 (segment (start 108.204 100.3592) (end 111.9416 100.3592) (width 0.4) (layer B.Cu) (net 4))
 (segment (start 111.9416 100.3592) (end 112.014 100.4316) (width 0.4) (layer B.Cu) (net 4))
 (segment (start 117.3292 99.7864) (end 112.6592 99.7864) (width 0.4) (layer B.Cu) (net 4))
 (segment (start 112.6592 99.7864) (end 112.014 100.4316) (width 0.4) (layer B.Cu) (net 4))
 (segment (start 112.014 95.3516) (end 112.014 91.36) (width 0.4) (layer B.Cu) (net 5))
 (segment (start 112.014 91.36) (end 112.4928 90.8812) (width 0.4) (layer B.Cu) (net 5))
 (segment (start 112.014 95.3516) (end 116.7348 95.3516) (width 0.4) (layer B.Cu) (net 5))
 (segment (start 116.7348 95.3516) (end 117.38 94.7064) (width 0.4) (layer B.Cu) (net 5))
 (segment (start 117.491 85.791) (end 112.837 85.791) (width 0.4) (layer B.Cu) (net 6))
 (segment (start 112.837 85.791) (end 112.141 86.487) (width 0.4) (layer B.Cu) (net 6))
 (segment (start 108.077 90.09) (end 108.077 89.99) (width 0.4) (layer B.Cu) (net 6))
 (segment (start 108.077 89.99) (end 111.58 86.487) (width 0.4) (layer B.Cu) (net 6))
 (segment (start 111.58 86.487) (end 112.141 86.487) (width 0.4) (layer B.Cu) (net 6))
 (segment (start 108.077 80.565) (end 111.299 80.565) (width 0.4) (layer B.Cu) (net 7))
 (segment (start 111.299 80.565) (end 112.141 81.407) (width 0.4) (layer B.Cu) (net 7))
 (segment (start 117.348 80.391) (end 113.157 80.391) (width 0.4) (layer B.Cu) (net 7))
 (segment (start 113.157 80.391) (end 112.141 81.407) (width 0.4) (layer B.Cu) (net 7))
 (segment (start 108.077 114.888) (end 110.664 114.888) (width 0.4) (layer B.Cu) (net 8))
 (segment (start 110.664 114.888) (end 112.141 113.411) (width 0.4) (layer B.Cu) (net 8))
 (segment (start 117.634 112.334) (end 113.218 112.334) (width 0.4) (layer B.Cu) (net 8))
 (segment (start 113.218 112.334) (end 112.141 113.411) (width 0.4) (layer B.Cu) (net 8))
 (segment (start 117.491 106.746) (end 113.726 106.746) (width 0.4) (layer B.Cu) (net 9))
 (segment (start 113.726 106.746) (end 112.141 108.331) (width 0.4) (layer B.Cu) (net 9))
 (segment (start 108.204 106.854) (end 110.664 106.854) (width 0.4) (layer B.Cu) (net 9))
 (segment (start 110.664 106.854) (end 112.141 108.331) (width 0.4) (layer B.Cu) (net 9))
 (segment (start 124.634 91.3892) (end 124.634 95.17) (width 0.4) (layer B.Cu) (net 10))
 (segment (start 124.634 95.17) (end 124.968 95.504) (width 0.4) (layer B.Cu) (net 10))
 (segment (start 119.38 95.6564) (end 124.8156 95.6564) (width 0.4) (layer B.Cu) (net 10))
 (segment (start 124.8156 95.6564) (end 124.968 95.504) (width 0.4) (layer B.Cu) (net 10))
 (segment (start 124.9896 104.1908) (end 124.9896 100.6056) (width 0.4) (layer B.Cu) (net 11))
 (segment (start 124.9896 100.6056) (end 124.968 100.584) (width 0.4) (layer B.Cu) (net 11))
 (segment (start 119.3292 100.7364) (end 124.8156 100.7364) (width 0.4) (layer B.Cu) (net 11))
 (segment (start 124.8156 100.7364) (end 124.968 100.584) (width 0.4) (layer B.Cu) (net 11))
 (segment (start 128.651 81.073) (end 125.683 81.073) (width 0.4) (layer B.Cu) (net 12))
 (segment (start 125.683 81.073) (end 124.968 81.788) (width 0.4) (layer B.Cu) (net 12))
 (segment (start 119.348 81.341) (end 124.521 81.341) (width 0.4) (layer B.Cu) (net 12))
 (segment (start 124.521 81.341) (end 124.968 81.788) (width 0.4) (layer B.Cu) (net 12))
 (segment (start 119.491 107.696) (end 124.333 107.696) (width 0.4) (layer B.Cu) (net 14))
 (segment (start 124.333 107.696) (end 124.841 108.204) (width 0.4) (layer B.Cu) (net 14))
 (segment (start 128.651 109.554) (end 126.191 109.554) (width 0.4) (layer B.Cu) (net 14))
 (segment (start 126.191 109.554) (end 124.841 108.204) (width 0.4) (layer B.Cu) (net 14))
 (segment (start 128.651 114.761) (end 126.318 114.761) (width 0.4) (layer B.Cu) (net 15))
 (segment (start 126.318 114.761) (end 124.841 113.284) (width 0.4) (layer B.Cu) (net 15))
 (segment (start 124.841 113.284) (end 122.71968 113.284) (width 0.4) (layer B.Cu) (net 15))
 (segment (start 122.71968 113.284) (end 119.634 113.284) (width 0.4) (layer B.Cu) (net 15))
 (segment (start 119.491 86.741) (end 124.841 86.741) (width 0.4) (layer B.Cu) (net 13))
 (segment (start 124.841 86.741) (end 124.968 86.868) (width 0.4) (layer B.Cu) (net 13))
 (segment (start 128.651 86.2) (end 125.636 86.2) (width 0.4) (layer B.Cu) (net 13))
 (segment (start 125.636 86.2) (end 124.968 86.868) (width 0.4) (layer B.Cu) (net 13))
 (segment (start 114.554 71.962) (end 114.554 74.248) (width 0.4) (layer B.Cu) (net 16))
 (segment (start 114.554 74.248) (end 114.728 74.422) (width 0.4) (layer B.Cu) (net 16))
 (segment (start 114.427 61.802) (end 114.427 64.723) (width 0.4) (layer B.Cu) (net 17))
 (segment (start 114.427 64.723) (end 114.601 64.897) (width 0.4) (layer B.Cu) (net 17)))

